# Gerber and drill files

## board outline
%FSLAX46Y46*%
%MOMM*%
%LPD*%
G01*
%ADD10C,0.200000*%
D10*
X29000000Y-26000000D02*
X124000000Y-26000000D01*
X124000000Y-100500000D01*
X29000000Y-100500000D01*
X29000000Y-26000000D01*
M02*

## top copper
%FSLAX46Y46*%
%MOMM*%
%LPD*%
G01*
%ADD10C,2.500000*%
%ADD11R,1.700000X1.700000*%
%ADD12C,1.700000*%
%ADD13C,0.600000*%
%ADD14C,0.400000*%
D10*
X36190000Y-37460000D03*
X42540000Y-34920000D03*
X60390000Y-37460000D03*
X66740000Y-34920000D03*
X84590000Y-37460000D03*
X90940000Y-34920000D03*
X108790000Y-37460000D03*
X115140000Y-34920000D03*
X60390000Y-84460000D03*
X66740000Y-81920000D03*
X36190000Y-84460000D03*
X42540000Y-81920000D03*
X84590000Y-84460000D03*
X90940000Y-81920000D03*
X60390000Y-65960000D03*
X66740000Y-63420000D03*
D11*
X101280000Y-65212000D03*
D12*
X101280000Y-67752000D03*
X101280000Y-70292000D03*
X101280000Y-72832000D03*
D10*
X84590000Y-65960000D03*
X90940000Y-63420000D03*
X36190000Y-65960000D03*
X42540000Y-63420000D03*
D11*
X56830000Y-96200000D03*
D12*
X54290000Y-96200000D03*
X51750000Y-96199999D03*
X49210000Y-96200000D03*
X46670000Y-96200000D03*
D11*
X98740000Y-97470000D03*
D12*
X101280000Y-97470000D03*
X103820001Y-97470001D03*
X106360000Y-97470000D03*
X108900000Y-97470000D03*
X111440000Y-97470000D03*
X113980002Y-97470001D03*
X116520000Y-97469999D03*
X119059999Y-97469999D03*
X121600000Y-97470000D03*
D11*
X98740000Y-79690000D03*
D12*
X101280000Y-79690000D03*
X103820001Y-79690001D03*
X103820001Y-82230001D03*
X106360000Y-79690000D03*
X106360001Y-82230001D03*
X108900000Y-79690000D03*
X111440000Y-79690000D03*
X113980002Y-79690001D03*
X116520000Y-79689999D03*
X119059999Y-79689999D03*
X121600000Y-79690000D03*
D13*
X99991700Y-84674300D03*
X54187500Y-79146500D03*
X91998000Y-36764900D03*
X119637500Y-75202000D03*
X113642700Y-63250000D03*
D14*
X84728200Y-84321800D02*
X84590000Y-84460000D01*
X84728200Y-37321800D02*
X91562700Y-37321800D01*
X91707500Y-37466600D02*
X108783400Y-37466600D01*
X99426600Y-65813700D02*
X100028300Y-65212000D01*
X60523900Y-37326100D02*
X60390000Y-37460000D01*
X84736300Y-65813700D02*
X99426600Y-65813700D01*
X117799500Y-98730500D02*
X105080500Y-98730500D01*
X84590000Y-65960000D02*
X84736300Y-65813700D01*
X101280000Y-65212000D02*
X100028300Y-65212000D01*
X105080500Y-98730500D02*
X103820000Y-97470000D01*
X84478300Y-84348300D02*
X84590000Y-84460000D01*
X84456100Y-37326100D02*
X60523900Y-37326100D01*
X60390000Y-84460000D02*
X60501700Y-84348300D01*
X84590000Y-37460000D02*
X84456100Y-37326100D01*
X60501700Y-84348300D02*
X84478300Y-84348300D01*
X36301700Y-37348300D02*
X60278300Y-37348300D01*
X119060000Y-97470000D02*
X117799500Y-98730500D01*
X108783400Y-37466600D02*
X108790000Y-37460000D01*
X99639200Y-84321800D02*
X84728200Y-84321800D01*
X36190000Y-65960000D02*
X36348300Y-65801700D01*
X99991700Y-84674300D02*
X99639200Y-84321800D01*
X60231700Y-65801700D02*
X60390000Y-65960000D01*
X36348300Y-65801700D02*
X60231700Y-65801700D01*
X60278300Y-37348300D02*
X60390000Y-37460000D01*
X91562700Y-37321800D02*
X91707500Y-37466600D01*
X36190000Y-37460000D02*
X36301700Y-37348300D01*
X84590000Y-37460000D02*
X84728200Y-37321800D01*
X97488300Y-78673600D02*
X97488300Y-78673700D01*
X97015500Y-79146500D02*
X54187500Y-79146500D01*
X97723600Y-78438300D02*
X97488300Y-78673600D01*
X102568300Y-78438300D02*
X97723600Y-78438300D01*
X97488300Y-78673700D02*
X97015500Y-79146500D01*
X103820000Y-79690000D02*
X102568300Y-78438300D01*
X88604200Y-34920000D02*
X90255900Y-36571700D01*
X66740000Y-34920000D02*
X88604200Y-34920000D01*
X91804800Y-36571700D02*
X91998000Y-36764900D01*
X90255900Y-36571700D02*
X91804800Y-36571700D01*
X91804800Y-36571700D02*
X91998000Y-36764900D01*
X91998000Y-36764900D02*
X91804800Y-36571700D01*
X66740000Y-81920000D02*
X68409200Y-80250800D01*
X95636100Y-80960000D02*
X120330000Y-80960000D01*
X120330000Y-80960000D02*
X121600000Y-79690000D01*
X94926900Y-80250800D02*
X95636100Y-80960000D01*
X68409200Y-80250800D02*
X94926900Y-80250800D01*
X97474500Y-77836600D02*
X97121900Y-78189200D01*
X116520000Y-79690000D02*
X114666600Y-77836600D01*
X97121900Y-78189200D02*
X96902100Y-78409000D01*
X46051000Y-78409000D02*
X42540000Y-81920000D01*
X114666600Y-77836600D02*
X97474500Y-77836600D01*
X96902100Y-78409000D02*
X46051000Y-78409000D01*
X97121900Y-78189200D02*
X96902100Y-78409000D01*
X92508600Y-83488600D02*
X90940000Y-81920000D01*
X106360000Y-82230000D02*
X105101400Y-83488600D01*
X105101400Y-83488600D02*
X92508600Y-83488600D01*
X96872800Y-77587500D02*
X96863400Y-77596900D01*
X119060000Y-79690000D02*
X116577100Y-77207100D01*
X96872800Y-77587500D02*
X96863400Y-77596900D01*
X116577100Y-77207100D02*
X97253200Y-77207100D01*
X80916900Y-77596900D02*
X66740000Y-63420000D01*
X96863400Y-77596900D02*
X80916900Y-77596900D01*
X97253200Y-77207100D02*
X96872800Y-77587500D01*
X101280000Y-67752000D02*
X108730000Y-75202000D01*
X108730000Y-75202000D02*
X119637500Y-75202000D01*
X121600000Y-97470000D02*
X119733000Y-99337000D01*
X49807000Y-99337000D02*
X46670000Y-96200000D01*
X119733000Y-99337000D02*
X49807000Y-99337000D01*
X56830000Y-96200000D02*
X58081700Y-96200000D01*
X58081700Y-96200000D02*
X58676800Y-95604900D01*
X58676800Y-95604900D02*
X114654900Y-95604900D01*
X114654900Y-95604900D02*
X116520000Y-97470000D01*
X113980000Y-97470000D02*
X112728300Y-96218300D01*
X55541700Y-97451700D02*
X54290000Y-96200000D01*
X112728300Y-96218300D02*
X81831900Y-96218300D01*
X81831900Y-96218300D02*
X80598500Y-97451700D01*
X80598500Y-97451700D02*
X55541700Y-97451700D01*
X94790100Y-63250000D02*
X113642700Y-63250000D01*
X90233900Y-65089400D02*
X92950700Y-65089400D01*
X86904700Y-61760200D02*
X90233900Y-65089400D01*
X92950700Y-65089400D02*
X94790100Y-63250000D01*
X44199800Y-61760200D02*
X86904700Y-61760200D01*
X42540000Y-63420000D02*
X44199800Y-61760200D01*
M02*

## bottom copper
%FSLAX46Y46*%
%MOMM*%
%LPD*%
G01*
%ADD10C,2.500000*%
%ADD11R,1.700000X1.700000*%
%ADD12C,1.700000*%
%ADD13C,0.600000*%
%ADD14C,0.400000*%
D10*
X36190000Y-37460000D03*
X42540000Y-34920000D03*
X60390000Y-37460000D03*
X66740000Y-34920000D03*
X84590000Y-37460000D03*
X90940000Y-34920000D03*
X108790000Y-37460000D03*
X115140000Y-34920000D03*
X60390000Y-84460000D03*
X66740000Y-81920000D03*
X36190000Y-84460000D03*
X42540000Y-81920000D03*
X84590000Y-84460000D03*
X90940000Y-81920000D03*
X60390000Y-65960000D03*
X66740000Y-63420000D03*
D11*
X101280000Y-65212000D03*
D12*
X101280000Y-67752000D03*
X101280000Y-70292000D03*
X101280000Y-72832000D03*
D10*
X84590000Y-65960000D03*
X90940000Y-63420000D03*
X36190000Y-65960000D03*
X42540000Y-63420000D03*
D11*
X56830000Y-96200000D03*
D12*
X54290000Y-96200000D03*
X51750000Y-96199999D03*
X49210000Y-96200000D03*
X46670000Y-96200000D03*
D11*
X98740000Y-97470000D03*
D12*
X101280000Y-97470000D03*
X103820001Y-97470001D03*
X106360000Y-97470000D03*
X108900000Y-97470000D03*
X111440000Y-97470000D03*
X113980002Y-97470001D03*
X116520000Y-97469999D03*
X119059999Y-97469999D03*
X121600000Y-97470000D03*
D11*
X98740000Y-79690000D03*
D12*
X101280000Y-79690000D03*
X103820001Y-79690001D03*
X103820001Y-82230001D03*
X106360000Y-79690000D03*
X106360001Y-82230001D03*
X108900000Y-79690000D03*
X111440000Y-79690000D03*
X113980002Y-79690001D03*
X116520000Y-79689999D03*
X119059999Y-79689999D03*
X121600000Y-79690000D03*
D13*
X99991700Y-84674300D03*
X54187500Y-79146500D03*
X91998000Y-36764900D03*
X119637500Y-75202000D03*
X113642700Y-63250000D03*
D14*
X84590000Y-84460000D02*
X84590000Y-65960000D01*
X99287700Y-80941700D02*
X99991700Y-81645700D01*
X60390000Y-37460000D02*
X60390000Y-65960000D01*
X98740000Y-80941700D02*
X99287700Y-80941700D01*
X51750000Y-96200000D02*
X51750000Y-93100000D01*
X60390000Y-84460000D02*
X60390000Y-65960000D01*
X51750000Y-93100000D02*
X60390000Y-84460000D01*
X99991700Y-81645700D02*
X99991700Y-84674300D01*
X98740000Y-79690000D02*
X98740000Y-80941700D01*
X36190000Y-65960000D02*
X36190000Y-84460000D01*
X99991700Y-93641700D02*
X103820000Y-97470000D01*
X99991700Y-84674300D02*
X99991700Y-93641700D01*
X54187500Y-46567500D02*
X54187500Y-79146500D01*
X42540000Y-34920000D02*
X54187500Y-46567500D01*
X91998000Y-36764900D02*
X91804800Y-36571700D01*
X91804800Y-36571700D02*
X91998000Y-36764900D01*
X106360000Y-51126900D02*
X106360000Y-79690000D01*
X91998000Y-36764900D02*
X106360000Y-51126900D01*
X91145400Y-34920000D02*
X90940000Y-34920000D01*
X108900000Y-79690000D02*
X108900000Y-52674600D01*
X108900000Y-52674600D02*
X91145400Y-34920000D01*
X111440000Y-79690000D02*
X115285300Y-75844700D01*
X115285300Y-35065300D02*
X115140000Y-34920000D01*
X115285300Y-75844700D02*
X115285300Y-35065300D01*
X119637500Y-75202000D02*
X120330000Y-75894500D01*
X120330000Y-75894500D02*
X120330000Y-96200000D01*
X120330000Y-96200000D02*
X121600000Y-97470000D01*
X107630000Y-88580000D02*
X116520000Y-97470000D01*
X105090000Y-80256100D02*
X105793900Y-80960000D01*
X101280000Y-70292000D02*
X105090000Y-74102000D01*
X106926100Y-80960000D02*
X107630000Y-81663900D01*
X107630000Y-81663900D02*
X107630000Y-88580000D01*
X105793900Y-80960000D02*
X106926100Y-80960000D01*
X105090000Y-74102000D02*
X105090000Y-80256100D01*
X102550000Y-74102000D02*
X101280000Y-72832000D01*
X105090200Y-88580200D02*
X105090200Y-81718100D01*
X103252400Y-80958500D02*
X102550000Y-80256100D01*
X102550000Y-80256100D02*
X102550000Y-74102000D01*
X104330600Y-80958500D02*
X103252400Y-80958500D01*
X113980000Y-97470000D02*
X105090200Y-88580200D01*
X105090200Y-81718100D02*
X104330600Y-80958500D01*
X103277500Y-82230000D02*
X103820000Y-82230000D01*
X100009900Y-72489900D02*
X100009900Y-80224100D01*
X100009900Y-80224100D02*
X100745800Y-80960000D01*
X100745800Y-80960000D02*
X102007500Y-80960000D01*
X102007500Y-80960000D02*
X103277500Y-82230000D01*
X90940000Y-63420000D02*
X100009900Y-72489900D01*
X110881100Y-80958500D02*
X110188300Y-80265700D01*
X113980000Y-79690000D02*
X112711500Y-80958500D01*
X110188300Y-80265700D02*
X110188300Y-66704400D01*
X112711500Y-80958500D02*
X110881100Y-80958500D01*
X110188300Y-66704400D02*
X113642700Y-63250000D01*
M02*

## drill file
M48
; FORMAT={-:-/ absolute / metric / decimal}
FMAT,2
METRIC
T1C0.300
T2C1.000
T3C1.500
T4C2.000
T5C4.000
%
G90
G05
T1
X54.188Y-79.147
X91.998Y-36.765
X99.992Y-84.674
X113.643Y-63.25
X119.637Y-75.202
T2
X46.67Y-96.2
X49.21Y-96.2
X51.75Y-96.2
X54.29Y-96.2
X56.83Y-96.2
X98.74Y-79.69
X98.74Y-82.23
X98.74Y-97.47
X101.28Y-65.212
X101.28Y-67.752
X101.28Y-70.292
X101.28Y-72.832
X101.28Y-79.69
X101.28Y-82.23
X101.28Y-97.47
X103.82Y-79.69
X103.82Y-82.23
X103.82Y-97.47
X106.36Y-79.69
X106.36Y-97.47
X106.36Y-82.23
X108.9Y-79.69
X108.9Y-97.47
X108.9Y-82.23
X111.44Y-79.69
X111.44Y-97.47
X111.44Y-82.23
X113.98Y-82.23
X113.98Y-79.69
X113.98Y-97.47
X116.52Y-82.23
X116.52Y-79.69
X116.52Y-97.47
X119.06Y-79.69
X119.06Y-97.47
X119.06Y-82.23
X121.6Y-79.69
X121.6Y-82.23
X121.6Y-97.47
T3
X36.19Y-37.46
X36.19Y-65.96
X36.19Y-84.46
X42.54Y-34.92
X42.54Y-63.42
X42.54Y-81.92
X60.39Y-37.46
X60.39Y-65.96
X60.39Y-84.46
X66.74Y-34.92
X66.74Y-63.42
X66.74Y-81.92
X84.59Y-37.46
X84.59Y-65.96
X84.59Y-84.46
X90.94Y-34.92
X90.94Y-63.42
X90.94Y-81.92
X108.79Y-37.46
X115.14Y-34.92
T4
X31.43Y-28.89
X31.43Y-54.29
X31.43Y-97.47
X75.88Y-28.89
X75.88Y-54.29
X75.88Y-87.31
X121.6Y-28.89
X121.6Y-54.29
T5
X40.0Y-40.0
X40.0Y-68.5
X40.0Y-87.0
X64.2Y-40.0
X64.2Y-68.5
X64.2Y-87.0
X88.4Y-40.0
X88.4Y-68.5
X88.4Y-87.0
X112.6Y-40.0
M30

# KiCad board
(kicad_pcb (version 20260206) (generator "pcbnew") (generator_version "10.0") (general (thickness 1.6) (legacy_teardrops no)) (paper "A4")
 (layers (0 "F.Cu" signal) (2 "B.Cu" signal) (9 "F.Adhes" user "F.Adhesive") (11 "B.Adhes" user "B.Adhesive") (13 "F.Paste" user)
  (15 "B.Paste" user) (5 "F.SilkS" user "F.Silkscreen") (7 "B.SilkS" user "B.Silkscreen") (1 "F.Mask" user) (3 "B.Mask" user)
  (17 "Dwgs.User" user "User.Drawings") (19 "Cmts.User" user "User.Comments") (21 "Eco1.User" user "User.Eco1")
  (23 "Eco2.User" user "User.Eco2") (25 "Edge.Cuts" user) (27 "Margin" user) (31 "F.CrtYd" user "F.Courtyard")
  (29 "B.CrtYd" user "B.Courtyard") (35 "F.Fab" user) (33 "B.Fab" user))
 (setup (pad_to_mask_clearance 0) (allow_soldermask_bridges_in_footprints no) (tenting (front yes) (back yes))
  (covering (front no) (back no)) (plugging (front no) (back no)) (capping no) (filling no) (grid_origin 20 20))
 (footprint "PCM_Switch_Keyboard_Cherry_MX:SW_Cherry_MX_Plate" (layer "F.Cu") (at 40 40)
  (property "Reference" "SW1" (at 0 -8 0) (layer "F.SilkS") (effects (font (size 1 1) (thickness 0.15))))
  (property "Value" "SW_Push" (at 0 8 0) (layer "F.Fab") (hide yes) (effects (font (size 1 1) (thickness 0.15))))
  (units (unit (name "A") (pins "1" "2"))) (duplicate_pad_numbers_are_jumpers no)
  (pad "" np_thru_hole circle (at 0 0) (size 4 4) (drill 4) (layers "*.Cu" "*.Mask"))
  (pad "1" thru_hole circle (at -3.81 -2.54) (size 2.5 2.5) (drill 1.5) (layers "*.Cu" "*.Mask") (remove_unused_layers no) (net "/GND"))
  (pad "2" thru_hole circle (at 2.54 -5.08) (size 2.5 2.5) (drill 1.5) (layers "*.Cu" "*.Mask") (remove_unused_layers no) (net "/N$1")))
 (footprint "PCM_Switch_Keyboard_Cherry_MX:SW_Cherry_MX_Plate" (layer "F.Cu") (at 64.2 40)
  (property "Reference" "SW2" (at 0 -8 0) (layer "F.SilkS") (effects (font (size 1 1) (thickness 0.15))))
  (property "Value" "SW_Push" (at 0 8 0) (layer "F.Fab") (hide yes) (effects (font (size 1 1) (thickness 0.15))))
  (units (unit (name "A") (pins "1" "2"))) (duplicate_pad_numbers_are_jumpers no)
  (pad "" np_thru_hole circle (at 0 0) (size 4 4) (drill 4) (layers "*.Cu" "*.Mask"))
  (pad "1" thru_hole circle (at -3.81 -2.54) (size 2.5 2.5) (drill 1.5) (layers "*.Cu" "*.Mask") (remove_unused_layers no) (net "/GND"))
  (pad "2" thru_hole circle (at 2.54 -5.08) (size 2.5 2.5) (drill 1.5) (layers "*.Cu" "*.Mask") (remove_unused_layers no) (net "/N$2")))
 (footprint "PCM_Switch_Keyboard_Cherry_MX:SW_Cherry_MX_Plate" (layer "F.Cu") (at 88.4 40)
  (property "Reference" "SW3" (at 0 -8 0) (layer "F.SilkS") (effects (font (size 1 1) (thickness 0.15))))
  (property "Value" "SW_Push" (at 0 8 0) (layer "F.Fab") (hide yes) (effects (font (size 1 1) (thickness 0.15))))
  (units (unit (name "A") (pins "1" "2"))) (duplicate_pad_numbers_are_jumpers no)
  (pad "" np_thru_hole circle (at 0 0) (size 4 4) (drill 4) (layers "*.Cu" "*.Mask"))
  (pad "1" thru_hole circle (at -3.81 -2.54) (size 2.5 2.5) (drill 1.5) (layers "*.Cu" "*.Mask") (remove_unused_layers no) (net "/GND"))
  (pad "2" thru_hole circle (at 2.54 -5.08) (size 2.5 2.5) (drill 1.5) (layers "*.Cu" "*.Mask") (remove_unused_layers no) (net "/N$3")))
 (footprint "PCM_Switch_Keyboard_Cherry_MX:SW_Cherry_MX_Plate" (layer "F.Cu") (at 112.6 40)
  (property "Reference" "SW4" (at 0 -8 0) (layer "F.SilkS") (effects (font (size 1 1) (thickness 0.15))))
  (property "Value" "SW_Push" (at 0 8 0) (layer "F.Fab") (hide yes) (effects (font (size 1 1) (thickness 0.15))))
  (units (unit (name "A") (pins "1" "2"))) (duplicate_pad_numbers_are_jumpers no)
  (pad "" np_thru_hole circle (at 0 0) (size 4 4) (drill 4) (layers "*.Cu" "*.Mask"))
  (pad "1" thru_hole circle (at -3.81 -2.54) (size 2.5 2.5) (drill 1.5) (layers "*.Cu" "*.Mask") (remove_unused_layers no) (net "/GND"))
  (pad "2" thru_hole circle (at 2.54 -5.08) (size 2.5 2.5) (drill 1.5) (layers "*.Cu" "*.Mask") (remove_unused_layers no) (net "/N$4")))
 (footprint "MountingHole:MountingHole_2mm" (layer "F.Cu") (at 75.88 28.89 90)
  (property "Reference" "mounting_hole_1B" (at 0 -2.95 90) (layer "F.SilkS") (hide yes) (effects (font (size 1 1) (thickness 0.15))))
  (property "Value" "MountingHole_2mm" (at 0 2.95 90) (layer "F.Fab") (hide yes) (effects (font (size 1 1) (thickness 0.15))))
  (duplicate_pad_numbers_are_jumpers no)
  (pad "" np_thru_hole circle (at 0 0 90) (size 2 2) (drill 2) (layers "*.Cu" "*.Mask")))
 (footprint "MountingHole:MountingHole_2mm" (layer "F.Cu") (at 31.43 28.89 90)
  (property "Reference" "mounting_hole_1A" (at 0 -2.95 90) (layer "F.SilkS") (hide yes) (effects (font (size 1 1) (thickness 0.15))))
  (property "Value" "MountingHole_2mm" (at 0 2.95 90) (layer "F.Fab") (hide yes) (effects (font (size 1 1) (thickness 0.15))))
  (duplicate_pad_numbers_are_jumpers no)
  (pad "" np_thru_hole circle (at 0 0 90) (size 2 2) (drill 2) (layers "*.Cu" "*.Mask")))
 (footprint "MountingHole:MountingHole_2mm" (layer "F.Cu") (at 75.88 54.29 90)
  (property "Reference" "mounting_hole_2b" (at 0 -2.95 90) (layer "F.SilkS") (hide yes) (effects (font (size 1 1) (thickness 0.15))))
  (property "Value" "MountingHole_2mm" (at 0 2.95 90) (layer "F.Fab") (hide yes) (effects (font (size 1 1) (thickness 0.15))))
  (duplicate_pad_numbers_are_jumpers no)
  (pad "" np_thru_hole circle (at 0 0 90) (size 2 2) (drill 2) (layers "*.Cu" "*.Mask")))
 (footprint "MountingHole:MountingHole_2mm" (layer "F.Cu") (at 31.43 54.29 90)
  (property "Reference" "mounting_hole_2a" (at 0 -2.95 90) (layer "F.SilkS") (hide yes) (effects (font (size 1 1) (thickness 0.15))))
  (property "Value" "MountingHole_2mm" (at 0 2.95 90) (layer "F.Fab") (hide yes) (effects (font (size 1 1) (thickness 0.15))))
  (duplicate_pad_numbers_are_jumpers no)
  (pad "" np_thru_hole circle (at 0 0 90) (size 2 2) (drill 2) (layers "*.Cu" "*.Mask")))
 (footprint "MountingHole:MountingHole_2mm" (layer "F.Cu") (at 121.6 28.89 90)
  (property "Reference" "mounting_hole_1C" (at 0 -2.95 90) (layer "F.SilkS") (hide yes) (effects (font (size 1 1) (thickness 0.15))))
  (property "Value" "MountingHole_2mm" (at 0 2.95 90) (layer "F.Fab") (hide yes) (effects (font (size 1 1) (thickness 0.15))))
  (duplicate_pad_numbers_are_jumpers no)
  (pad "" np_thru_hole circle (at 0 0 90) (size 2 2) (drill 2) (layers "*.Cu" "*.Mask")))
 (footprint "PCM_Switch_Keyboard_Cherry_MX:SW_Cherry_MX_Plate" (layer "F.Cu") (at 64.2 87)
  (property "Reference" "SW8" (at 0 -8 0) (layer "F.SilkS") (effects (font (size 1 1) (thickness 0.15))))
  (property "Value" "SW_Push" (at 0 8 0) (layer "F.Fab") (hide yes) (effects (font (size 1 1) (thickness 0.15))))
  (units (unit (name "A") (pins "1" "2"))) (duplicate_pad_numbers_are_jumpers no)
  (pad "" np_thru_hole circle (at 0 0) (size 4 4) (drill 4) (layers "*.Cu" "*.Mask"))
  (pad "1" thru_hole circle (at -3.81 -2.54) (size 2.5 2.5) (drill 1.5) (layers "*.Cu" "*.Mask") (remove_unused_layers no) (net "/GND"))
  (pad "2" thru_hole circle (at 2.54 -5.08) (size 2.5 2.5) (drill 1.5) (layers "*.Cu" "*.Mask") (remove_unused_layers no) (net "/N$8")))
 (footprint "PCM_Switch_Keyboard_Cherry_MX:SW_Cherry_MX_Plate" (layer "F.Cu") (at 40 87)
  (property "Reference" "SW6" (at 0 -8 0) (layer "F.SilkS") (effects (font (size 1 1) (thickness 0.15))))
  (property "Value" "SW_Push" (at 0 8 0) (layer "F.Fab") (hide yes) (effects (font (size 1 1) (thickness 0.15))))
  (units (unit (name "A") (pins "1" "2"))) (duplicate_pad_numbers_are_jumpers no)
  (pad "" np_thru_hole circle (at 0 0) (size 4 4) (drill 4) (layers "*.Cu" "*.Mask"))
  (pad "1" thru_hole circle (at -3.81 -2.54) (size 2.5 2.5) (drill 1.5) (layers "*.Cu" "*.Mask") (remove_unused_layers no) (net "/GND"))
  (pad "2" thru_hole circle (at 2.54 -5.08) (size 2.5 2.5) (drill 1.5) (layers "*.Cu" "*.Mask") (remove_unused_layers no) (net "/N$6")))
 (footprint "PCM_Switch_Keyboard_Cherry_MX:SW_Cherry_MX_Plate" (layer "F.Cu") (at 88.4 87)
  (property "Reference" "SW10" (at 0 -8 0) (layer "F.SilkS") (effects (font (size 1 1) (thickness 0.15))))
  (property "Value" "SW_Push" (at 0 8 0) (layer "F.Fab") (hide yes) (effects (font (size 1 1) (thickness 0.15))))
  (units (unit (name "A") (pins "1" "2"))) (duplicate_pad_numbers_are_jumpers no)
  (pad "" np_thru_hole circle (at 0 0) (size 4 4) (drill 4) (layers "*.Cu" "*.Mask"))
  (pad "1" thru_hole circle (at -3.81 -2.54) (size 2.5 2.5) (drill 1.5) (layers "*.Cu" "*.Mask") (remove_unused_layers no) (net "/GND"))
  (pad "2" thru_hole circle (at 2.54 -5.08) (size 2.5 2.5) (drill 1.5) (layers "*.Cu" "*.Mask") (remove_unused_layers no) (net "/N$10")))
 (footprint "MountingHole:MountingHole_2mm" (layer "F.Cu") (at 75.88 87.31 90)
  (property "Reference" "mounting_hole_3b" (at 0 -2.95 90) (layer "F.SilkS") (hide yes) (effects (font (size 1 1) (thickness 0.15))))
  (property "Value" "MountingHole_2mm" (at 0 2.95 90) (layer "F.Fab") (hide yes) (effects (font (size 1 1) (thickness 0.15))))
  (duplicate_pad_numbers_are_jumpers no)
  (pad "" np_thru_hole circle (at 0 0 90) (size 2 2) (drill 2) (layers "*.Cu" "*.Mask")))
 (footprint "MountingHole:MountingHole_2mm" (layer "F.Cu") (at 121.6 54.29 90)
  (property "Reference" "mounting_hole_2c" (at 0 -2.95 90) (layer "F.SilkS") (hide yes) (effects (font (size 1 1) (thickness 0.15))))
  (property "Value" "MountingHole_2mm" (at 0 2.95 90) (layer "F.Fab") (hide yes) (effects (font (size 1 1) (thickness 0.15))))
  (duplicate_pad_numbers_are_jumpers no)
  (pad "" np_thru_hole circle (at 0 0 90) (size 2 2) (drill 2) (layers "*.Cu" "*.Mask")))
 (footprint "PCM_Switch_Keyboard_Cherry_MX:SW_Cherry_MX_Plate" (layer "F.Cu") (at 64.2 68.5)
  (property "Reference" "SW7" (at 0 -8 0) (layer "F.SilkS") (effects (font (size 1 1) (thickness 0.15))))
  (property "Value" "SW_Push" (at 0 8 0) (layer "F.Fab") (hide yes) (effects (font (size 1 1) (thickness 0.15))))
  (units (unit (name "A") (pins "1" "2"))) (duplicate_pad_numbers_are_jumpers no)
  (pad "" np_thru_hole circle (at 0 0) (size 4 4) (drill 4) (layers "*.Cu" "*.Mask"))
  (pad "1" thru_hole circle (at -3.81 -2.54) (size 2.5 2.5) (drill 1.5) (layers "*.Cu" "*.Mask") (remove_unused_layers no) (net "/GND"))
  (pad "2" thru_hole circle (at 2.54 -5.08) (size 2.5 2.5) (drill 1.5) (layers "*.Cu" "*.Mask") (remove_unused_layers no) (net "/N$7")))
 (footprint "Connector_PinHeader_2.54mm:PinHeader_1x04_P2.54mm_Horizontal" (layer "F.Cu") (at 101.28 65.212)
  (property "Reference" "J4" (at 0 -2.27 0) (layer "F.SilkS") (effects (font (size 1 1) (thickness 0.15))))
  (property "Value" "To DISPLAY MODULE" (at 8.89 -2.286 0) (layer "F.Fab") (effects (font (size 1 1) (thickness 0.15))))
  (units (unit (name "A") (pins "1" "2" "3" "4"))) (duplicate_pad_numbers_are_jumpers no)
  (pad "1" thru_hole rect (at 0 0) (size 1.7 1.7) (drill 1) (layers "*.Cu" "*.Mask") (remove_unused_layers no) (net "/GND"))
  (pad "2" thru_hole circle (at 0 2.54) (size 1.7 1.7) (drill 1) (layers "*.Cu" "*.Mask") (remove_unused_layers no) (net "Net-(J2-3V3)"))
  (pad "3" thru_hole circle (at 0 5.08) (size 1.7 1.7) (drill 1) (layers "*.Cu" "*.Mask") (remove_unused_layers no) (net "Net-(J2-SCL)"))
  (pad "4" thru_hole circle (at 0 7.62) (size 1.7 1.7) (drill 1) (layers "*.Cu" "*.Mask") (remove_unused_layers no) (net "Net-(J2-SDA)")))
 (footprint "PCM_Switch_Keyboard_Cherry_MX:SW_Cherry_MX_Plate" (layer "F.Cu") (at 88.4 68.5)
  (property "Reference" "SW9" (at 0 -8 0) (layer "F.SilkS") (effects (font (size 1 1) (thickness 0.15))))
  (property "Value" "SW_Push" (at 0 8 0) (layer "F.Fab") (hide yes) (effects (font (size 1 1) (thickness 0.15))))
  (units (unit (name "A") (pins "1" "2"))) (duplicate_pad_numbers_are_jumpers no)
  (pad "" np_thru_hole circle (at 0 0) (size 4 4) (drill 4) (layers "*.Cu" "*.Mask"))
  (pad "1" thru_hole circle (at -3.81 -2.54) (size 2.5 2.5) (drill 1.5) (layers "*.Cu" "*.Mask") (remove_unused_layers no) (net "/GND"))
  (pad "2" thru_hole circle (at 2.54 -5.08) (size 2.5 2.5) (drill 1.5) (layers "*.Cu" "*.Mask") (remove_unused_layers no) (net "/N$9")))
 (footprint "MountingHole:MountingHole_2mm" (layer "F.Cu") (at 31.43 97.47 90)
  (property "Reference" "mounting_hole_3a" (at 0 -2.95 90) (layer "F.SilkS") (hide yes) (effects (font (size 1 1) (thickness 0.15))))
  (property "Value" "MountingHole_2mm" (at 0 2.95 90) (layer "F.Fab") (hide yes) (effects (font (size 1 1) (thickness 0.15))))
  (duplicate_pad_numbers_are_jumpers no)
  (pad "" np_thru_hole circle (at 0 0 90) (size 2 2) (drill 2) (layers "*.Cu" "*.Mask")))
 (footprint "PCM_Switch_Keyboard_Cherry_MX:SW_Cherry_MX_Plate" (layer "F.Cu") (at 40 68.5)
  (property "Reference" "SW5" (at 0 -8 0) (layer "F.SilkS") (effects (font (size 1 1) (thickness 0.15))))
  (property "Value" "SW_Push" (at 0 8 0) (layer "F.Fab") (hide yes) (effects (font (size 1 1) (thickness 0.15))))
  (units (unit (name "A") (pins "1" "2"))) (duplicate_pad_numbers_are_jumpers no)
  (pad "" np_thru_hole circle (at 0 0) (size 4 4) (drill 4) (layers "*.Cu" "*.Mask"))
  (pad "1" thru_hole circle (at -3.81 -2.54) (size 2.5 2.5) (drill 1.5) (layers "*.Cu" "*.Mask") (remove_unused_layers no) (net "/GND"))
  (pad "2" thru_hole circle (at 2.54 -5.08) (size 2.5 2.5) (drill 1.5) (layers "*.Cu" "*.Mask") (remove_unused_layers no) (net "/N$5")))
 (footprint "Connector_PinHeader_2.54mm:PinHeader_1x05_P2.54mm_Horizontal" (layer "B.Cu") (at 56.83 96.2 90)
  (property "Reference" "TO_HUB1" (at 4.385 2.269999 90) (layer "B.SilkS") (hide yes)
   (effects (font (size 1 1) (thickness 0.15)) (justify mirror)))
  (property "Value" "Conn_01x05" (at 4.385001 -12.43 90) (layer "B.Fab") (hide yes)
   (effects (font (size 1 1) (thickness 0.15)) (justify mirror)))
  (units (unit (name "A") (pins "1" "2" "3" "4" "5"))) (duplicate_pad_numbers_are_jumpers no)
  (pad "1" thru_hole rect (at 0 0 90) (size 1.7 1.7) (drill 1) (layers "*.Cu" "*.Mask") (remove_unused_layers no) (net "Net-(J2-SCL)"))
  (pad "2" thru_hole circle (at 0 -2.54 90) (size 1.7 1.7) (drill 1) (layers "*.Cu" "*.Mask") (remove_unused_layers no) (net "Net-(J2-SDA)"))
  (pad "3" thru_hole circle (at 0.000001 -5.08 90) (size 1.7 1.7) (drill 1) (layers "*.Cu" "*.Mask") (remove_unused_layers no) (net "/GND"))
  (pad "4" thru_hole circle (at 0 -7.62 90) (size 1.7 1.7) (drill 1) (layers "*.Cu" "*.Mask") (remove_unused_layers no)
   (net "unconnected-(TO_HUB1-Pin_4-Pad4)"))
  (pad "5" thru_hole circle (at 0 -10.16 90) (size 1.7 1.7) (drill 1) (layers "*.Cu" "*.Mask") (remove_unused_layers no)
   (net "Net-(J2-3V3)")))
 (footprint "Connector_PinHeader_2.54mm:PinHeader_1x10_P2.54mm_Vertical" (layer "B.Cu") (at 98.74 97.47 -90)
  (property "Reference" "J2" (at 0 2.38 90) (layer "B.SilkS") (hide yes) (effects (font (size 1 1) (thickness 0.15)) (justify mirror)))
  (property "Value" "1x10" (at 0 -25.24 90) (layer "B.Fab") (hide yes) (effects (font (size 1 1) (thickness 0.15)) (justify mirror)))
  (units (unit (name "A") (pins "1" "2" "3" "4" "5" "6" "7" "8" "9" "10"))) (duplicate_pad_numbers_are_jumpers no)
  (pad "1" thru_hole rect (at 0 0 270) (size 1.7 1.7) (drill 1) (layers "*.Cu" "*.Mask") (remove_unused_layers no)
   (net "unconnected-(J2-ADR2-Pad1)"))
  (pad "2" thru_hole circle (at 0 -2.54 270) (size 1.7 1.7) (drill 1) (layers "*.Cu" "*.Mask") (remove_unused_layers no)
   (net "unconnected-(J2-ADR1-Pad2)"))
  (pad "3" thru_hole circle (at 0.000001 -5.080001 270) (size 1.7 1.7) (drill 1) (layers "*.Cu" "*.Mask") (remove_unused_layers no)
   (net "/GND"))
  (pad "4" thru_hole circle (at 0 -7.62 270) (size 1.7 1.7) (drill 1) (layers "*.Cu" "*.Mask") (remove_unused_layers no)
   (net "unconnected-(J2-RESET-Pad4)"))
  (pad "5" thru_hole circle (at 0 -10.16 270) (size 1.7 1.7) (drill 1) (layers "*.Cu" "*.Mask") (remove_unused_layers no)
   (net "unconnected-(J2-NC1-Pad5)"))
  (pad "6" thru_hole circle (at 0 -12.7 270) (size 1.7 1.7) (drill 1) (layers "*.Cu" "*.Mask") (remove_unused_layers no)
   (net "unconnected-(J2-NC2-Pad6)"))
  (pad "7" thru_hole circle (at 0.000001 -15.240002 270) (size 1.7 1.7) (drill 1) (layers "*.Cu" "*.Mask") (remove_unused_layers no)
   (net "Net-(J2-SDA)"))
  (pad "8" thru_hole circle (at -0.000001 -17.78 270) (size 1.7 1.7) (drill 1) (layers "*.Cu" "*.Mask") (remove_unused_layers no)
   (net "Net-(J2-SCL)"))
  (pad "9" thru_hole circle (at -0.000001 -20.319999 270) (size 1.7 1.7) (drill 1) (layers "*.Cu" "*.Mask") (remove_unused_layers no)
   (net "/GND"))
  (pad "10" thru_hole circle (at 0 -22.86 270) (size 1.7 1.7) (drill 1) (layers "*.Cu" "*.Mask") (remove_unused_layers no)
   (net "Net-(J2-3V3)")))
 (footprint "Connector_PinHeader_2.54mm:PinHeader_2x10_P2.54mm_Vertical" (layer "B.Cu") (at 98.74 79.69 -90)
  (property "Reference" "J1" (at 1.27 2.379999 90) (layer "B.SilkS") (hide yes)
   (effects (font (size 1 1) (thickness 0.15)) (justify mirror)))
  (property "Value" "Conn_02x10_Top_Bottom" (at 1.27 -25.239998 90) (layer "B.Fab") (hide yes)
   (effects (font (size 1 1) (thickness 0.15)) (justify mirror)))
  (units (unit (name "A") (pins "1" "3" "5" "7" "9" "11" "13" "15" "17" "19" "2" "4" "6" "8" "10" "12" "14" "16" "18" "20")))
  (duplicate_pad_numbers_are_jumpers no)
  (pad "1" thru_hole rect (at 0 0 270) (size 1.7 1.7) (drill 1) (layers "*.Cu" "*.Mask") (remove_unused_layers no) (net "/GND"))
  (pad "2" thru_hole circle (at 2.54 0 270) (size 1.7 1.7) (drill 1) (layers "*.Cu" "*.Mask") (remove_unused_layers yes)
   (keep_end_layers no) (zone_layer_connections) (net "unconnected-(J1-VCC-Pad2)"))
  (pad "3" thru_hole circle (at 0 -2.54 270) (size 1.7 1.7) (drill 1) (layers "*.Cu" "*.Mask") (remove_unused_layers no)
   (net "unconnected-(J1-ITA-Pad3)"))
  (pad "4" thru_hole circle (at 2.54 -2.54 270) (size 1.7 1.7) (drill 1) (layers "*.Cu" "*.Mask") (remove_unused_layers yes)
   (keep_end_layers no) (zone_layer_connections) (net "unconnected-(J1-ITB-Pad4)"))
  (pad "5" thru_hole circle (at 0.000001 -5.080001 270) (size 1.7 1.7) (drill 1) (layers "*.Cu" "*.Mask") (remove_unused_layers no)
   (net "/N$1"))
  (pad "6" thru_hole circle (at 2.540001 -5.080001 270) (size 1.7 1.7) (drill 1) (layers "*.Cu" "*.Mask") (remove_unused_layers no)
   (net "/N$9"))
  (pad "7" thru_hole circle (at 0 -7.62 270) (size 1.7 1.7) (drill 1) (layers "*.Cu" "*.Mask") (remove_unused_layers no) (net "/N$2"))
  (pad "8" thru_hole circle (at 2.540001 -7.620001 270) (size 1.7 1.7) (drill 1) (layers "*.Cu" "*.Mask") (remove_unused_layers no)
   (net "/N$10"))
  (pad "9" thru_hole circle (at 0 -10.16 270) (size 1.7 1.7) (drill 1) (layers "*.Cu" "*.Mask") (remove_unused_layers no) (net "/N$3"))
  (pad "10" thru_hole circle (at 2.540001 -10.160001 270) (size 1.7 1.7) (drill 1) (layers "*.Cu" "*.Mask") (remove_unused_layers yes)
   (keep_end_layers no) (zone_layer_connections) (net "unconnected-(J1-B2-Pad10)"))
  (pad "11" thru_hole circle (at 0 -12.7 270) (size 1.7 1.7) (drill 1) (layers "*.Cu" "*.Mask") (remove_unused_layers no) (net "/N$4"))
  (pad "12" thru_hole circle (at 2.540001 -12.700002 270) (size 1.7 1.7) (drill 1) (layers "*.Cu" "*.Mask") (remove_unused_layers yes)
   (keep_end_layers no) (zone_layer_connections) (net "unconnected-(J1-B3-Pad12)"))
  (pad "13" thru_hole circle (at 0.000001 -15.240002 270) (size 1.7 1.7) (drill 1) (layers "*.Cu" "*.Mask") (remove_unused_layers no)
   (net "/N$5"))
  (pad "14" thru_hole circle (at 2.54 -15.24 270) (size 1.7 1.7) (drill 1) (layers "*.Cu" "*.Mask") (remove_unused_layers yes)
   (keep_end_layers no) (zone_layer_connections) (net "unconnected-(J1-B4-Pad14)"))
  (pad "15" thru_hole circle (at -0.000001 -17.78 270) (size 1.7 1.7) (drill 1) (layers "*.Cu" "*.Mask") (remove_unused_layers no)
   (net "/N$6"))
  (pad "16" thru_hole circle (at 2.540001 -17.779999 270) (size 1.7 1.7) (drill 1) (layers "*.Cu" "*.Mask") (remove_unused_layers yes)
   (keep_end_layers no) (zone_layer_connections) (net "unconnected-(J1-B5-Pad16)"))
  (pad "17" thru_hole circle (at -0.000001 -20.319999 270) (size 1.7 1.7) (drill 1) (layers "*.Cu" "*.Mask") (remove_unused_layers no)
   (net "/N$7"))
  (pad "18" thru_hole circle (at 2.539998 -20.320001 270) (size 1.7 1.7) (drill 1) (layers "*.Cu" "*.Mask") (remove_unused_layers yes)
   (keep_end_layers no) (zone_layer_connections) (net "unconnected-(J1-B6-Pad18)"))
  (pad "19" thru_hole circle (at 0 -22.86 270) (size 1.7 1.7) (drill 1) (layers "*.Cu" "*.Mask") (remove_unused_layers no) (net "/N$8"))
  (pad "20" thru_hole circle (at 2.539998 -22.86 270) (size 1.7 1.7) (drill 1) (layers "*.Cu" "*.Mask") (remove_unused_layers yes)
   (keep_end_layers no) (zone_layer_connections) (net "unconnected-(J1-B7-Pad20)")))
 (gr_rect (start 29 26) (end 124 100.5) (stroke (width 0.2) (type solid)) (fill no) (layer "Edge.Cuts"))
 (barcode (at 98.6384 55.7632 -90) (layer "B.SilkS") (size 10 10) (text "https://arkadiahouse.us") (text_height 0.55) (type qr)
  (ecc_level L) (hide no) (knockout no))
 (segment (start 84.7282 84.3218) (end 84.59 84.46) (width 0.4) (layer "F.Cu") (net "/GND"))
 (segment (start 84.7282 37.3218) (end 91.5627 37.3218) (width 0.4) (layer "F.Cu") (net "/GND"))
 (segment (start 91.7075 37.4666) (end 108.7834 37.4666) (width 0.4) (layer "F.Cu") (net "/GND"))
 (segment (start 99.4266 65.8137) (end 100.0283 65.212) (width 0.4) (layer "F.Cu") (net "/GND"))
 (segment (start 60.5239 37.3261) (end 60.39 37.46) (width 0.4) (layer "F.Cu") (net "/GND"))
 (segment (start 84.7363 65.8137) (end 99.4266 65.8137) (width 0.4) (layer "F.Cu") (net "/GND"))
 (segment (start 117.7995 98.7305) (end 105.0805 98.7305) (width 0.4) (layer "F.Cu") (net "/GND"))
 (segment (start 84.59 65.96) (end 84.7363 65.8137) (width 0.4) (layer "F.Cu") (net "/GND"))
 (segment (start 101.28 65.212) (end 100.0283 65.212) (width 0.4) (layer "F.Cu") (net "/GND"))
 (segment (start 105.0805 98.7305) (end 103.82 97.47) (width 0.4) (layer "F.Cu") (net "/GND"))
 (segment (start 84.4783 84.3483) (end 84.59 84.46) (width 0.4) (layer "F.Cu") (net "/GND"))
 (segment (start 84.4561 37.3261) (end 60.5239 37.3261) (width 0.4) (layer "F.Cu") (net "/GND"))
 (segment (start 60.39 84.46) (end 60.5017 84.3483) (width 0.4) (layer "F.Cu") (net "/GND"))
 (segment (start 84.59 37.46) (end 84.4561 37.3261) (width 0.4) (layer "F.Cu") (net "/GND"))
 (segment (start 60.5017 84.3483) (end 84.4783 84.3483) (width 0.4) (layer "F.Cu") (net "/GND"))
 (segment (start 36.3017 37.3483) (end 60.2783 37.3483) (width 0.4) (layer "F.Cu") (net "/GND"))
 (segment (start 119.06 97.47) (end 117.7995 98.7305) (width 0.4) (layer "F.Cu") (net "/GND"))
 (segment (start 108.7834 37.4666) (end 108.79 37.46) (width 0.4) (layer "F.Cu") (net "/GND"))
 (segment (start 99.6392 84.3218) (end 84.7282 84.3218) (width 0.4) (layer "F.Cu") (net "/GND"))
 (segment (start 36.19 65.96) (end 36.3483 65.8017) (width 0.4) (layer "F.Cu") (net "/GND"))
 (segment (start 99.9917 84.6743) (end 99.6392 84.3218) (width 0.4) (layer "F.Cu") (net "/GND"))
 (segment (start 60.2317 65.8017) (end 60.39 65.96) (width 0.4) (layer "F.Cu") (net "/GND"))
 (segment (start 36.3483 65.8017) (end 60.2317 65.8017) (width 0.4) (layer "F.Cu") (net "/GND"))
 (segment (start 60.2783 37.3483) (end 60.39 37.46) (width 0.4) (layer "F.Cu") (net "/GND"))
 (segment (start 91.5627 37.3218) (end 91.7075 37.4666) (width 0.4) (layer "F.Cu") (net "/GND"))
 (segment (start 36.19 37.46) (end 36.3017 37.3483) (width 0.4) (layer "F.Cu") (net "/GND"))
 (segment (start 84.59 37.46) (end 84.7282 37.3218) (width 0.4) (layer "F.Cu") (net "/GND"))
 (via (at 99.9917 84.6743) (size 0.6) (drill 0.3) (layers "F.Cu" "B.Cu") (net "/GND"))
 (segment (start 84.59 84.46) (end 84.59 65.96) (width 0.4) (layer "B.Cu") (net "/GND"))
 (segment (start 99.2877 80.9417) (end 99.9917 81.6457) (width 0.4) (layer "B.Cu") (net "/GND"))
 (segment (start 60.39 37.46) (end 60.39 65.96) (width 0.4) (layer "B.Cu") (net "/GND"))
 (segment (start 98.74 80.9417) (end 99.2877 80.9417) (width 0.4) (layer "B.Cu") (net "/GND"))
 (segment (start 51.75 96.2) (end 51.75 93.1) (width 0.4) (layer "B.Cu") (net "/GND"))
 (segment (start 60.39 84.46) (end 60.39 65.96) (width 0.4) (layer "B.Cu") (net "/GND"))
 (segment (start 51.75 93.1) (end 60.39 84.46) (width 0.4) (layer "B.Cu") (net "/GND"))
 (segment (start 99.9917 81.6457) (end 99.9917 84.6743) (width 0.4) (layer "B.Cu") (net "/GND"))
 (segment (start 98.74 79.69) (end 98.74 80.9417) (width 0.4) (layer "B.Cu") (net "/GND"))
 (segment (start 36.19 65.96) (end 36.19 84.46) (width 0.4) (layer "B.Cu") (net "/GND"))
 (segment (start 99.9917 93.6417) (end 103.82 97.47) (width 0.4) (layer "B.Cu") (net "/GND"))
 (segment (start 99.9917 84.6743) (end 99.9917 93.6417) (width 0.4) (layer "B.Cu") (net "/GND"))
 (segment (start 97.4883 78.6736) (end 97.4883 78.6737) (width 0.4) (layer "F.Cu") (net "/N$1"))
 (segment (start 97.0155 79.1465) (end 54.1875 79.1465) (width 0.4) (layer "F.Cu") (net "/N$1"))
 (segment (start 97.7236 78.4383) (end 97.4883 78.6736) (width 0.4) (layer "F.Cu") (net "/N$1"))
 (segment (start 102.5683 78.4383) (end 97.7236 78.4383) (width 0.4) (layer "F.Cu") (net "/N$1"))
 (segment (start 97.4883 78.6737) (end 97.0155 79.1465) (width 0.4) (layer "F.Cu") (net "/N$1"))
 (segment (start 103.82 79.69) (end 102.5683 78.4383) (width 0.4) (layer "F.Cu") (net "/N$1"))
 (via (at 54.1875 79.1465) (size 0.6) (drill 0.3) (layers "F.Cu" "B.Cu") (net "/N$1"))
 (segment (start 54.1875 46.5675) (end 54.1875 79.1465) (width 0.4) (layer "B.Cu") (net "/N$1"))
 (segment (start 42.54 34.92) (end 54.1875 46.5675) (width 0.4) (layer "B.Cu") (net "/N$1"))
 (segment (start 88.6042 34.92) (end 90.2559 36.5717) (width 0.4) (layer "F.Cu") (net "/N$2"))
 (segment (start 66.74 34.92) (end 88.6042 34.92) (width 0.4) (layer "F.Cu") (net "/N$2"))
 (segment (start 91.8048 36.5717) (end 91.998 36.7649) (width 0.4) (layer "F.Cu") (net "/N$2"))
 (segment (start 90.2559 36.5717) (end 91.8048 36.5717) (width 0.4) (layer "F.Cu") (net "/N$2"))
 (segment (start 91.8048 36.5717) (end 91.998 36.7649) (width 0.4) (layer "F.Cu") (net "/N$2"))
 (segment (start 91.998 36.7649) (end 91.8048 36.5717) (width 0.4) (layer "F.Cu") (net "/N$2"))
 (via (at 91.998 36.7649) (size 0.6) (drill 0.3) (layers "F.Cu" "B.Cu") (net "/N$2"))
 (segment (start 91.998 36.7649) (end 91.8048 36.5717) (width 0.4) (layer "B.Cu") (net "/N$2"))
 (segment (start 91.8048 36.5717) (end 91.998 36.7649) (width 0.4) (layer "B.Cu") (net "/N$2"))
 (segment (start 106.36 51.1269) (end 106.36 79.69) (width 0.4) (layer "B.Cu") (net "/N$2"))
 (segment (start 91.998 36.7649) (end 106.36 51.1269) (width 0.4) (layer "B.Cu") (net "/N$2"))
 (segment (start 91.1454 34.92) (end 90.94 34.92) (width 0.4) (layer "B.Cu") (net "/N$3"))
 (segment (start 108.9 79.69) (end 108.9 52.6746) (width 0.4) (layer "B.Cu") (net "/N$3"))
 (segment (start 108.9 52.6746) (end 91.1454 34.92) (width 0.4) (layer "B.Cu") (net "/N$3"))
 (segment (start 111.44 79.69) (end 115.2853 75.8447) (width 0.4) (layer "B.Cu") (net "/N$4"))
 (segment (start 115.2853 35.0653) (end 115.14 34.92) (width 0.4) (layer "B.Cu") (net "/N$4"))
 (segment (start 115.2853 75.8447) (end 115.2853 35.0653) (width 0.4) (layer "B.Cu") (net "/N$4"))
 (segment (start 66.74 81.92) (end 68.4092 80.2508) (width 0.4) (layer "F.Cu") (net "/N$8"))
 (segment (start 95.6361 80.96) (end 120.33 80.96) (width 0.4) (layer "F.Cu") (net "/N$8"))
 (segment (start 120.33 80.96) (end 121.6 79.69) (width 0.4) (layer "F.Cu") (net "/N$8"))
 (segment (start 94.9269 80.2508) (end 95.6361 80.96) (width 0.4) (layer "F.Cu") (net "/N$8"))
 (segment (start 68.4092 80.2508) (end 94.9269 80.2508) (width 0.4) (layer "F.Cu") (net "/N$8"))
 (segment (start 97.4745 77.8366) (end 97.1219 78.1892) (width 0.4) (layer "F.Cu") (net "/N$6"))
 (segment (start 116.52 79.69) (end 114.6666 77.8366) (width 0.4) (layer "F.Cu") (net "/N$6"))
 (segment (start 97.1219 78.1892) (end 96.9021 78.409) (width 0.4) (layer "F.Cu") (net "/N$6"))
 (segment (start 46.051 78.409) (end 42.54 81.92) (width 0.4) (layer "F.Cu") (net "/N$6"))
 (segment (start 114.6666 77.8366) (end 97.4745 77.8366) (width 0.4) (layer "F.Cu") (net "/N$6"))
 (segment (start 96.9021 78.409) (end 46.051 78.409) (width 0.4) (layer "F.Cu") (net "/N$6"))
 (segment (start 97.1219 78.1892) (end 96.9021 78.409) (width 0.4) (layer "F.Cu") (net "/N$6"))
 (segment (start 92.5086 83.4886) (end 90.94 81.92) (width 0.4) (layer "F.Cu") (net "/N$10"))
 (segment (start 106.36 82.23) (end 105.1014 83.4886) (width 0.4) (layer "F.Cu") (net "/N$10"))
 (segment (start 105.1014 83.4886) (end 92.5086 83.4886) (width 0.4) (layer "F.Cu") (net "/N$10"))
 (segment (start 96.8728 77.5875) (end 96.8634 77.5969) (width 0.4) (layer "F.Cu") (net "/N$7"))
 (segment (start 119.06 79.69) (end 116.5771 77.2071) (width 0.4) (layer "F.Cu") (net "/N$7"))
 (segment (start 96.8728 77.5875) (end 96.8634 77.5969) (width 0.4) (layer "F.Cu") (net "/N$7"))
 (segment (start 116.5771 77.2071) (end 97.2532 77.2071) (width 0.4) (layer "F.Cu") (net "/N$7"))
 (segment (start 80.9169 77.5969) (end 66.74 63.42) (width 0.4) (layer "F.Cu") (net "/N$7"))
 (segment (start 96.8634 77.5969) (end 80.9169 77.5969) (width 0.4) (layer "F.Cu") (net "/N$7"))
 (segment (start 97.2532 77.2071) (end 96.8728 77.5875) (width 0.4) (layer "F.Cu") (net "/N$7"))
 (segment (start 101.28 67.752) (end 108.73 75.202) (width 0.4) (layer "F.Cu") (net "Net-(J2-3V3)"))
 (segment (start 108.73 75.202) (end 119.6375 75.202) (width 0.4) (layer "F.Cu") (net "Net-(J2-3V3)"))
 (segment (start 121.6 97.47) (end 119.733 99.337) (width 0.4) (layer "F.Cu") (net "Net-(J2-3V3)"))
 (segment (start 49.807 99.337) (end 46.67 96.2) (width 0.4) (layer "F.Cu") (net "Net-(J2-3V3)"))
 (segment (start 119.733 99.337) (end 49.807 99.337) (width 0.4) (layer "F.Cu") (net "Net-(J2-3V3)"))
 (via (at 119.6375 75.202) (size 0.6) (drill 0.3) (layers "F.Cu" "B.Cu") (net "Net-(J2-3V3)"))
 (segment (start 119.6375 75.202) (end 120.33 75.8945) (width 0.4) (layer "B.Cu") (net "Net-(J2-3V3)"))
 (segment (start 120.33 75.8945) (end 120.33 96.2) (width 0.4) (layer "B.Cu") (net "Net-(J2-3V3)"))
 (segment (start 120.33 96.2) (end 121.6 97.47) (width 0.4) (layer "B.Cu") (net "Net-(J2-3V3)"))
 (segment (start 56.83 96.2) (end 58.0817 96.2) (width 0.4) (layer "F.Cu") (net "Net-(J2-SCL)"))
 (segment (start 58.0817 96.2) (end 58.6768 95.6049) (width 0.4) (layer "F.Cu") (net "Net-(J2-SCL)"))
 (segment (start 58.6768 95.6049) (end 114.6549 95.6049) (width 0.4) (layer "F.Cu") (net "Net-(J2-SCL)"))
 (segment (start 114.6549 95.6049) (end 116.52 97.47) (width 0.4) (layer "F.Cu") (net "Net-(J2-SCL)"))
 (segment (start 107.63 88.58) (end 116.52 97.47) (width 0.4) (layer "B.Cu") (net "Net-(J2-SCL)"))
 (segment (start 105.09 80.2561) (end 105.7939 80.96) (width 0.4) (layer "B.Cu") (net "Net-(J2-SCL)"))
 (segment (start 101.28 70.292) (end 105.09 74.102) (width 0.4) (layer "B.Cu") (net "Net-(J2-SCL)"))
 (segment (start 106.9261 80.96) (end 107.63 81.6639) (width 0.4) (layer "B.Cu") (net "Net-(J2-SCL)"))
 (segment (start 107.63 81.6639) (end 107.63 88.58) (width 0.4) (layer "B.Cu") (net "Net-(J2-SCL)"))
 (segment (start 105.7939 80.96) (end 106.9261 80.96) (width 0.4) (layer "B.Cu") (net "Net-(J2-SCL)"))
 (segment (start 105.09 74.102) (end 105.09 80.2561) (width 0.4) (layer "B.Cu") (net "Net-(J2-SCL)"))
 (segment (start 113.98 97.47) (end 112.7283 96.2183) (width 0.4) (layer "F.Cu") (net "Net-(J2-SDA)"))
 (segment (start 55.5417 97.4517) (end 54.29 96.2) (width 0.4) (layer "F.Cu") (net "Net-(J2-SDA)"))
 (segment (start 112.7283 96.2183) (end 81.8319 96.2183) (width 0.4) (layer "F.Cu") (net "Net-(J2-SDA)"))
 (segment (start 81.8319 96.2183) (end 80.5985 97.4517) (width 0.4) (layer "F.Cu") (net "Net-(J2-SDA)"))
 (segment (start 80.5985 97.4517) (end 55.5417 97.4517) (width 0.4) (layer "F.Cu") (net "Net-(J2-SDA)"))
 (segment (start 102.55 74.102) (end 101.28 72.832) (width 0.4) (layer "B.Cu") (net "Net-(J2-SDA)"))
 (segment (start 105.0902 88.5802) (end 105.0902 81.7181) (width 0.4) (layer "B.Cu") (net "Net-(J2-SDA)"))
 (segment (start 103.2524 80.9585) (end 102.55 80.2561) (width 0.4) (layer "B.Cu") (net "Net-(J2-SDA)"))
 (segment (start 102.55 80.2561) (end 102.55 74.102) (width 0.4) (layer "B.Cu") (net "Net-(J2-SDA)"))
 (segment (start 104.3306 80.9585) (end 103.2524 80.9585) (width 0.4) (layer "B.Cu") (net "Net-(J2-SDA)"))
 (segment (start 113.98 97.47) (end 105.0902 88.5802) (width 0.4) (layer "B.Cu") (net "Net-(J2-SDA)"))
 (segment (start 105.0902 81.7181) (end 104.3306 80.9585) (width 0.4) (layer "B.Cu") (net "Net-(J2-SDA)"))
 (segment (start 103.2775 82.23) (end 103.82 82.23) (width 0.4) (layer "B.Cu") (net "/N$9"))
 (segment (start 100.0099 72.4899) (end 100.0099 80.2241) (width 0.4) (layer "B.Cu") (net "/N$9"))
 (segment (start 100.0099 80.2241) (end 100.7458 80.96) (width 0.4) (layer "B.Cu") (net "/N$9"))
 (segment (start 100.7458 80.96) (end 102.0075 80.96) (width 0.4) (layer "B.Cu") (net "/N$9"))
 (segment (start 102.0075 80.96) (end 103.2775 82.23) (width 0.4) (layer "B.Cu") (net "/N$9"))
 (segment (start 90.94 63.42) (end 100.0099 72.4899) (width 0.4) (layer "B.Cu") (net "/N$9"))
 (segment (start 94.7901 63.25) (end 113.6427 63.25) (width 0.4) (layer "F.Cu") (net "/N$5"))
 (segment (start 90.2339 65.0894) (end 92.9507 65.0894) (width 0.4) (layer "F.Cu") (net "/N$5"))
 (segment (start 86.9047 61.7602) (end 90.2339 65.0894) (width 0.4) (layer "F.Cu") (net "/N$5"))
 (segment (start 92.9507 65.0894) (end 94.7901 63.25) (width 0.4) (layer "F.Cu") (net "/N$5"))
 (segment (start 44.1998 61.7602) (end 86.9047 61.7602) (width 0.4) (layer "F.Cu") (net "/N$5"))
 (segment (start 42.54 63.42) (end 44.1998 61.7602) (width 0.4) (layer "F.Cu") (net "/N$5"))
 (via (at 113.6427 63.25) (size 0.6) (drill 0.3) (layers "F.Cu" "B.Cu") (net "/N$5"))
 (segment (start 110.8811 80.9585) (end 110.1883 80.2657) (width 0.4) (layer "B.Cu") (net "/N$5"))
 (segment (start 113.98 79.69) (end 112.7115 80.9585) (width 0.4) (layer "B.Cu") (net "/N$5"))
 (segment (start 110.1883 80.2657) (end 110.1883 66.7044) (width 0.4) (layer "B.Cu") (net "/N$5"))
 (segment (start 112.7115 80.9585) (end 110.8811 80.9585) (width 0.4) (layer "B.Cu") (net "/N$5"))
 (segment (start 110.1883 66.7044) (end 113.6427 63.25) (width 0.4) (layer "B.Cu") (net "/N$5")))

